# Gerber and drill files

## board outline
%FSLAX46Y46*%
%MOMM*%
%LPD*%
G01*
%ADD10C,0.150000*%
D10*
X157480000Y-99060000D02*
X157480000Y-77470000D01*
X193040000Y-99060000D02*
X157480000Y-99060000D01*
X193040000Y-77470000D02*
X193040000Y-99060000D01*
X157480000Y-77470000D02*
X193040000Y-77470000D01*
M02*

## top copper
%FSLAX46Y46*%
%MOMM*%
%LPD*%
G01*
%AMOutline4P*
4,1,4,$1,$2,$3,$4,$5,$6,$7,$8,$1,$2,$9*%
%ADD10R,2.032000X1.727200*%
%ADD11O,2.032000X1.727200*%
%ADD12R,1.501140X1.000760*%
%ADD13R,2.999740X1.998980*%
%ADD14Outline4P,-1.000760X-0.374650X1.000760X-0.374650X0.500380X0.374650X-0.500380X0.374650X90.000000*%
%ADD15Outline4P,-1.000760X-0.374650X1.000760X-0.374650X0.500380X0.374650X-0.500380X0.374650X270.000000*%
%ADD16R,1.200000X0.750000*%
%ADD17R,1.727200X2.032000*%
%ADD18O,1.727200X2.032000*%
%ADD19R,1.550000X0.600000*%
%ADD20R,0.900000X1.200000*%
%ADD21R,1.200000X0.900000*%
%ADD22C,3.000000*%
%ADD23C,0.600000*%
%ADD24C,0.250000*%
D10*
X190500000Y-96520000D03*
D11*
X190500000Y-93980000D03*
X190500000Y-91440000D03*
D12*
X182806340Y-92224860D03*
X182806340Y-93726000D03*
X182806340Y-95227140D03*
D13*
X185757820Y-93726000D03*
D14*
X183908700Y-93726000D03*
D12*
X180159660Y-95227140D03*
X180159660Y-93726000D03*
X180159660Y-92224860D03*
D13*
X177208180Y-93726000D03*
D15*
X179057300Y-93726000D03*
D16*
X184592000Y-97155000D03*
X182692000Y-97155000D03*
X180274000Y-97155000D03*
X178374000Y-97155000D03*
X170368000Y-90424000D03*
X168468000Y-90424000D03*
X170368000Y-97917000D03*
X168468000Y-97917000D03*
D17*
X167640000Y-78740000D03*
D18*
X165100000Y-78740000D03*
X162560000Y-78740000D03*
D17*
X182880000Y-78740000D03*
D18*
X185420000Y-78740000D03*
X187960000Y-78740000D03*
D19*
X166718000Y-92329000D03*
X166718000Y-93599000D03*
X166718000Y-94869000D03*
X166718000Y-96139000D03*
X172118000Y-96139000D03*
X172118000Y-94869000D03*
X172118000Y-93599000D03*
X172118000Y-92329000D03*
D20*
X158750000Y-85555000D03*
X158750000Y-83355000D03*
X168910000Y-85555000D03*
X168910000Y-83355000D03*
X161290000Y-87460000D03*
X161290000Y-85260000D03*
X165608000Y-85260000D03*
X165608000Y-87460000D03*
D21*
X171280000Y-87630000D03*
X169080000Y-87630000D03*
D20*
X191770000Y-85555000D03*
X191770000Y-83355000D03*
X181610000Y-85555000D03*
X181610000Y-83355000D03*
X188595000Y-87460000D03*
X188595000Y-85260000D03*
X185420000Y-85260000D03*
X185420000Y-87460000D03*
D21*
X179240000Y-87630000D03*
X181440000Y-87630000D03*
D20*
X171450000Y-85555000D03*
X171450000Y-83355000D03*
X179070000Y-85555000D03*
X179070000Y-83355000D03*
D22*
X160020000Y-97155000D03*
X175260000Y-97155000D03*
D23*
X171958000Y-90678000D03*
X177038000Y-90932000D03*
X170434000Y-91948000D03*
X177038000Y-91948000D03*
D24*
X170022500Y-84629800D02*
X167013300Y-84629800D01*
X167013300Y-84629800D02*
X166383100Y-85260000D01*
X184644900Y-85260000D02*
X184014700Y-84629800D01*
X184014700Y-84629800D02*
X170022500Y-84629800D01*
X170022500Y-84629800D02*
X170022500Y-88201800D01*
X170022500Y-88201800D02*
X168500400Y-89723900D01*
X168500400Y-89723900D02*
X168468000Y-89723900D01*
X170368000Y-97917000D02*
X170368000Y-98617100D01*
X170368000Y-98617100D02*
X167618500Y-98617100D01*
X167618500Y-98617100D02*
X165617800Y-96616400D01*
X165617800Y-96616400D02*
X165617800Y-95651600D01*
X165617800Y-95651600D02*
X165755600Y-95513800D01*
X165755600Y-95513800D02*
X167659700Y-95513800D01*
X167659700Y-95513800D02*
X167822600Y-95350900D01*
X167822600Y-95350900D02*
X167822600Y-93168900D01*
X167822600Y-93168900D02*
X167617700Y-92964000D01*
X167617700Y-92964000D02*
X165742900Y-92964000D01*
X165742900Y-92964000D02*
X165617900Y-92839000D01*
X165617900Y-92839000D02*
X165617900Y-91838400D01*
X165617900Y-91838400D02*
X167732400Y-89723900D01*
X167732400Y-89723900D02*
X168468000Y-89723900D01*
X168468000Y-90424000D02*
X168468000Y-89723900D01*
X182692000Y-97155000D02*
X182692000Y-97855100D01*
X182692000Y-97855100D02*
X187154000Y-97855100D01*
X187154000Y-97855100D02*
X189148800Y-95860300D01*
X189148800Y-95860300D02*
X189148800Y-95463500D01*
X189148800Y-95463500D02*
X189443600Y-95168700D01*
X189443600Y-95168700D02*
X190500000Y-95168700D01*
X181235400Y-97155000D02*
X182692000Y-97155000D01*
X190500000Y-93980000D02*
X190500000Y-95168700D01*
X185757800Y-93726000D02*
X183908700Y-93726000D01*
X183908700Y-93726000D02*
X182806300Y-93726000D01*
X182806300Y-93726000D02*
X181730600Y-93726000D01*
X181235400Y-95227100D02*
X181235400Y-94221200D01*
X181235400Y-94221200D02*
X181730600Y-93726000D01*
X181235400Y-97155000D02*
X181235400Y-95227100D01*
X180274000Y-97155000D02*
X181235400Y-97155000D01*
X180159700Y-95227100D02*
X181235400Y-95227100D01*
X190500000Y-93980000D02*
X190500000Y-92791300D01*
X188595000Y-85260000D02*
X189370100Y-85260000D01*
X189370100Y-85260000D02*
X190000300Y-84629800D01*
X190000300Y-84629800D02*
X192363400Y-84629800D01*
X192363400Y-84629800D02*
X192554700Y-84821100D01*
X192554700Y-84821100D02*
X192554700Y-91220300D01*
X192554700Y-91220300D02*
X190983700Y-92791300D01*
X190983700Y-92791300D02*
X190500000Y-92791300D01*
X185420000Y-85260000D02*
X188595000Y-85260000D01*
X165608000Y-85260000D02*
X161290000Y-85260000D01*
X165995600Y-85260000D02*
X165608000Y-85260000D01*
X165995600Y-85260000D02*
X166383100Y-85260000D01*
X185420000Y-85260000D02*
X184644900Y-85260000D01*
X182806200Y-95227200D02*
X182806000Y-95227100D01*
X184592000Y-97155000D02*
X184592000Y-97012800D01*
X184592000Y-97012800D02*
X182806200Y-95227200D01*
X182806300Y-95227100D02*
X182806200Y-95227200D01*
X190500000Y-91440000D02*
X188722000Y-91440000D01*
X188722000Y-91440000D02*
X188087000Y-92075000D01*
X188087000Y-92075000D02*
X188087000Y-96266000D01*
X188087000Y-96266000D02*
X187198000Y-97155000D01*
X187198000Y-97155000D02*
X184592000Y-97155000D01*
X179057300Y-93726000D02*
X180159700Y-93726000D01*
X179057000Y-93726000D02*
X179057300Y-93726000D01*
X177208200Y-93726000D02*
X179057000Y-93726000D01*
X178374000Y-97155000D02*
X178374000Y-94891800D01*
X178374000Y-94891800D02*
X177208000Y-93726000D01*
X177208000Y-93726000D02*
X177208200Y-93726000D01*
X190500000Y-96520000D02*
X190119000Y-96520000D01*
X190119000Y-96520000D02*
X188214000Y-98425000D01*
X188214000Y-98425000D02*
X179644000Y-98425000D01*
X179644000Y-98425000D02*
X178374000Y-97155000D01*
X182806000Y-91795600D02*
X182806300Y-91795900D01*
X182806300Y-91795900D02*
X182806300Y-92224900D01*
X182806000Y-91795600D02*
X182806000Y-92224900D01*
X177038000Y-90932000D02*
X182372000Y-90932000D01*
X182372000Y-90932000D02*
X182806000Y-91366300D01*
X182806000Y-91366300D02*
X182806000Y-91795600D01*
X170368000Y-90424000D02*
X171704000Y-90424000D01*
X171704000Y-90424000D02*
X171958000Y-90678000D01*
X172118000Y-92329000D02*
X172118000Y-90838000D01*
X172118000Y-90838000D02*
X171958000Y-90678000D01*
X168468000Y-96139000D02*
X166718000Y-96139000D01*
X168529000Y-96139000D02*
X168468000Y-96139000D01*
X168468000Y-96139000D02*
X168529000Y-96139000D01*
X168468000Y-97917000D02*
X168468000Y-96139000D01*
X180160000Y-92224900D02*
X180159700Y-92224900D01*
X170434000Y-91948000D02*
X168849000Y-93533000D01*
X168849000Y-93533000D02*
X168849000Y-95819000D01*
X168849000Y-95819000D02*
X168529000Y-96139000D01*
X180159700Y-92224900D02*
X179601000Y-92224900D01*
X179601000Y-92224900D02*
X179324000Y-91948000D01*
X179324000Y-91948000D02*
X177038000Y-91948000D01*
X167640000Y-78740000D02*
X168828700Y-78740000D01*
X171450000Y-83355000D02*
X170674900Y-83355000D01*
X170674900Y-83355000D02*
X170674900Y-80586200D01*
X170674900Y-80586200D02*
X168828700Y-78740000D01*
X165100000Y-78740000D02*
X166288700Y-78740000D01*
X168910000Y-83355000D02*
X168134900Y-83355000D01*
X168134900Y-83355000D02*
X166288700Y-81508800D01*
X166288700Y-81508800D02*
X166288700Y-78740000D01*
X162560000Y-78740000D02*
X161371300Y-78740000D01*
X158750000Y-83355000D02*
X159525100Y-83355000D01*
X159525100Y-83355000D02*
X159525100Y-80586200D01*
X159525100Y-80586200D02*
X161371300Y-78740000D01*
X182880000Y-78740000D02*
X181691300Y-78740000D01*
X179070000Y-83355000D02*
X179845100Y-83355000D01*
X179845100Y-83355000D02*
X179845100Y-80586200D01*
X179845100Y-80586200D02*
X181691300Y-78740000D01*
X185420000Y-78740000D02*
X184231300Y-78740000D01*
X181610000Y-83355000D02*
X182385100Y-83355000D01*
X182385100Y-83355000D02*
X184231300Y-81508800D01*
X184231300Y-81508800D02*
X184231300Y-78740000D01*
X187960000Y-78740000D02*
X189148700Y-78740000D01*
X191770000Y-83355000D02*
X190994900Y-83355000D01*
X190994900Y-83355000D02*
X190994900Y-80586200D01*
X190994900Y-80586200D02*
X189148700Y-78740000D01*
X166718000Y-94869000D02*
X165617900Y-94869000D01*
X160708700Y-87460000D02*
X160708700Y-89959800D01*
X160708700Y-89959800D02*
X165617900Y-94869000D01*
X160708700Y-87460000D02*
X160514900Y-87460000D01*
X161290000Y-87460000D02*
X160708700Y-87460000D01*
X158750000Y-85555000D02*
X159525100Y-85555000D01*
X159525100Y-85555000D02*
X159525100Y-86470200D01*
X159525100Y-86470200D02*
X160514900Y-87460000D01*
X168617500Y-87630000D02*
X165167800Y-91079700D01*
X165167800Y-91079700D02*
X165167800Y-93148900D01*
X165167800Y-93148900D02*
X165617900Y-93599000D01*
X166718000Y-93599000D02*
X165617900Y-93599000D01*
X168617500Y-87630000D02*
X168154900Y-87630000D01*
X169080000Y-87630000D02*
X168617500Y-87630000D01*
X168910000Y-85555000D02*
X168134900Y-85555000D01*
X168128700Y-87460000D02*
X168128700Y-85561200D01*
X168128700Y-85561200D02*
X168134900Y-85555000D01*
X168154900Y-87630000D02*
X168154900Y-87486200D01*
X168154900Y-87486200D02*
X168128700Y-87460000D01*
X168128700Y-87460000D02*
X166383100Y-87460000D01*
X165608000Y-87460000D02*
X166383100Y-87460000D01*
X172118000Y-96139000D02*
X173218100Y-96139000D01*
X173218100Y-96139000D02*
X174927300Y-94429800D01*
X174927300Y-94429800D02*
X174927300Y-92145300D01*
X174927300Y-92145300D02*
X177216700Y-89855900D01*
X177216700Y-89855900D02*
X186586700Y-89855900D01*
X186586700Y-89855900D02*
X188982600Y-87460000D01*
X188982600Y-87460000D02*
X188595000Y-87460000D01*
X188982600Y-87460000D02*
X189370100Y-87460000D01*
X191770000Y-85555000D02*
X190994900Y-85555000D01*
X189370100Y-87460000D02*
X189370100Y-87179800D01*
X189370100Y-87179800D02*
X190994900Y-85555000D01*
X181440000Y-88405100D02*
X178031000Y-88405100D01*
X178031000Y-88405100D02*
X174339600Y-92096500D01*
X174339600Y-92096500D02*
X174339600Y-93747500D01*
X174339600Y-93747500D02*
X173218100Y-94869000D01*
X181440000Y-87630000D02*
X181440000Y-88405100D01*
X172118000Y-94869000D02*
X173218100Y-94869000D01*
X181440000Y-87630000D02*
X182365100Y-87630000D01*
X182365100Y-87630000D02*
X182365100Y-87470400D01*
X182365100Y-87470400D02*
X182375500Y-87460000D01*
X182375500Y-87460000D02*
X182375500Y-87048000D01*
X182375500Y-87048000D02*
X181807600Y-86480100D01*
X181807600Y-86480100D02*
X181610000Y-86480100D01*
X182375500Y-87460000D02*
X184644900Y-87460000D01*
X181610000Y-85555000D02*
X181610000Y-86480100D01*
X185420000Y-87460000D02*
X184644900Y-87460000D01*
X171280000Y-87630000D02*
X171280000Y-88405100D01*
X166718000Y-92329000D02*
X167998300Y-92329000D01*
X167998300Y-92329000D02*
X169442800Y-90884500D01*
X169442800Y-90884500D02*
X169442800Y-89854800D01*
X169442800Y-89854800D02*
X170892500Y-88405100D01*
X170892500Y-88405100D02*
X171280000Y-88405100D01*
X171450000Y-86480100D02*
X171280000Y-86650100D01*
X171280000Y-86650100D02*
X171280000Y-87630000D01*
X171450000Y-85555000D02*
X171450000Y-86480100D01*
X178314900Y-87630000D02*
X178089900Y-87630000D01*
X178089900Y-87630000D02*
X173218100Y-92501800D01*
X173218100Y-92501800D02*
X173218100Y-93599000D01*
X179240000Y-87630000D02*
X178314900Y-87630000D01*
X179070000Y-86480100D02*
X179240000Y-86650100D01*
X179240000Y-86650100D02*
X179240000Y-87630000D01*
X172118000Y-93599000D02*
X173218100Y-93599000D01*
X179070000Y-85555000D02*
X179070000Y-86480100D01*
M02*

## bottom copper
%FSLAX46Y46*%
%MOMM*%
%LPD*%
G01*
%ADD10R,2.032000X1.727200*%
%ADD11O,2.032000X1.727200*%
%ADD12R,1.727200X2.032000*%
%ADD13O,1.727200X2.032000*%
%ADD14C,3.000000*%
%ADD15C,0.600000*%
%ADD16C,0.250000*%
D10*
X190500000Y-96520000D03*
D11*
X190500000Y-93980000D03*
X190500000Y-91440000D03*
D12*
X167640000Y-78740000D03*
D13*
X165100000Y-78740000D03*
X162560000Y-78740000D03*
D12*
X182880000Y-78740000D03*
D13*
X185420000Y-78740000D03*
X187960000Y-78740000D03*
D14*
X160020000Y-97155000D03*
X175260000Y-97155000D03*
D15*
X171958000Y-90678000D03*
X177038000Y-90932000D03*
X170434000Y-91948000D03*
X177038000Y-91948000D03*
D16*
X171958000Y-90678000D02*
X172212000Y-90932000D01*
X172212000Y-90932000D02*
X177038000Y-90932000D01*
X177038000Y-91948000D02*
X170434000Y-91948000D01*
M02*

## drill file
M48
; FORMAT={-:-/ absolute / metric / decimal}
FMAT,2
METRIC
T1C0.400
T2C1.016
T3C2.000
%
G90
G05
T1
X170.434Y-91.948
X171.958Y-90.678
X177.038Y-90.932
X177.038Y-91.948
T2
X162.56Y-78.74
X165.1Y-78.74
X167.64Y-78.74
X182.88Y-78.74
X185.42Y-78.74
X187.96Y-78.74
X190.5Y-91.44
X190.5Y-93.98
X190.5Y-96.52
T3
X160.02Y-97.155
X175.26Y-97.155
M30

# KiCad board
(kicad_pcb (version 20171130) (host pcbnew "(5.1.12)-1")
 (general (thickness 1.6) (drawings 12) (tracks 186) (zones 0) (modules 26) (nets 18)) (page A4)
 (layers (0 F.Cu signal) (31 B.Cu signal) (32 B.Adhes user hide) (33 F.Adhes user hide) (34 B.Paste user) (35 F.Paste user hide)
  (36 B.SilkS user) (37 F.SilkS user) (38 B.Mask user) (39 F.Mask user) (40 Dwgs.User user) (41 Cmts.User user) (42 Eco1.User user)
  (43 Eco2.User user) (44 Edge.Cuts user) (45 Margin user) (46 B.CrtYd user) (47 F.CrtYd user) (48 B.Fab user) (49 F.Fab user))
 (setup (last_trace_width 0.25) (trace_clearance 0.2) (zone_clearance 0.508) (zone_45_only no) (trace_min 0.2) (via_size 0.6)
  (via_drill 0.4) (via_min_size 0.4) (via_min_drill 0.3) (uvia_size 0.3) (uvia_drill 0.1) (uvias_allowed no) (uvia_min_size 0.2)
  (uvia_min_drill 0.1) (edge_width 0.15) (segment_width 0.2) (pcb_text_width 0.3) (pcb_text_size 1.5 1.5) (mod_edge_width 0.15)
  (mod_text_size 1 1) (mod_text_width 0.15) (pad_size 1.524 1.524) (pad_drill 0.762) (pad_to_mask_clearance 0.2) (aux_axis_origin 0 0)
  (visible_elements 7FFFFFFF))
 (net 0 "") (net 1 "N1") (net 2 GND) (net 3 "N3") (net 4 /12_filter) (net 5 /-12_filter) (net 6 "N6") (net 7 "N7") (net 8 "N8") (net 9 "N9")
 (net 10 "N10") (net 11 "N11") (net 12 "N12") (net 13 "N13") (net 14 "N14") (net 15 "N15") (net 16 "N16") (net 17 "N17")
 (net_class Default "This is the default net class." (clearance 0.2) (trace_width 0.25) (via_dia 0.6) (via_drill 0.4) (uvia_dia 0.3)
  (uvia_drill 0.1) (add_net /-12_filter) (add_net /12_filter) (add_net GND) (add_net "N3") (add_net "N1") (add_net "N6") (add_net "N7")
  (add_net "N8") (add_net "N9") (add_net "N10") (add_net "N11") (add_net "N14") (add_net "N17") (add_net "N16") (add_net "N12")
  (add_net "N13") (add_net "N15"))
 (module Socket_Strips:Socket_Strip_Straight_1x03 (layer F.Cu) (at 190.5 96.52 90)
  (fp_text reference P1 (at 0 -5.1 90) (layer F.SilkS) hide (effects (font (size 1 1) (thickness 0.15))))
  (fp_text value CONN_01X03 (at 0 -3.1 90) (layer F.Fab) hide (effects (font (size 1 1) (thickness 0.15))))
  (pad 1 thru_hole rect (at 0 0 90) (size 1.7272 2.032) (drill 1.016) (layers *.Cu *.Mask F.SilkS) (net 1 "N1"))
  (pad 2 thru_hole oval (at 2.54 0 90) (size 1.7272 2.032) (drill 1.016) (layers *.Cu *.Mask F.SilkS) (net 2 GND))
  (pad 3 thru_hole oval (at 5.08 0 90) (size 1.7272 2.032) (drill 1.016) (layers *.Cu *.Mask F.SilkS) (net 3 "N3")))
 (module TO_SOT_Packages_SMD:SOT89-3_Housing (layer F.Cu) (at 184.658 93.726 270)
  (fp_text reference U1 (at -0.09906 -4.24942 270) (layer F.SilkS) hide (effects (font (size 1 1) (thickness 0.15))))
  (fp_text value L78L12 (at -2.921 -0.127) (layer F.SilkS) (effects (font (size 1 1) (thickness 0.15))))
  (pad 1 smd rect (at -1.50114 1.85166 270) (size 1.00076 1.50114) (layers F.Cu F.Paste F.Mask) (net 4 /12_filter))
  (pad 2 smd rect (at 0 1.85166 270) (size 1.00076 1.50114) (layers F.Cu F.Paste F.Mask) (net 2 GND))
  (pad 3 smd rect (at 1.50114 1.85166 270) (size 1.00076 1.50114) (layers F.Cu F.Paste F.Mask) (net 3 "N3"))
  (pad 2 smd rect (at 0 -1.09982 270) (size 1.99898 2.99974) (layers F.Cu F.Paste F.Mask) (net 2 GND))
  (pad 2 smd trapezoid (at 0 0.7493 90) (size 1.50114 0.7493) (rect_delta 0 0.50038) (layers F.Cu F.Paste F.Mask) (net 2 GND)))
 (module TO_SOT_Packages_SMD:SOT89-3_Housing (layer F.Cu) (at 178.308 93.726 90)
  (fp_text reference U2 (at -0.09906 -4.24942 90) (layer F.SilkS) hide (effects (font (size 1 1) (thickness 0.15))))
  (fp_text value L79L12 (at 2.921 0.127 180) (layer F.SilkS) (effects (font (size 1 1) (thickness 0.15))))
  (pad 1 smd rect (at -1.50114 1.85166 90) (size 1.00076 1.50114) (layers F.Cu F.Paste F.Mask) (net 2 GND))
  (pad 2 smd rect (at 0 1.85166 90) (size 1.00076 1.50114) (layers F.Cu F.Paste F.Mask) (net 1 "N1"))
  (pad 3 smd rect (at 1.50114 1.85166 90) (size 1.00076 1.50114) (layers F.Cu F.Paste F.Mask) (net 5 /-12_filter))
  (pad 2 smd rect (at 0 -1.09982 90) (size 1.99898 2.99974) (layers F.Cu F.Paste F.Mask) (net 1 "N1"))
  (pad 2 smd trapezoid (at 0 0.7493 270) (size 1.50114 0.7493) (rect_delta 0 0.50038) (layers F.Cu F.Paste F.Mask) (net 1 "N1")))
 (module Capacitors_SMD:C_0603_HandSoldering (layer F.Cu) (at 183.642 97.155 180)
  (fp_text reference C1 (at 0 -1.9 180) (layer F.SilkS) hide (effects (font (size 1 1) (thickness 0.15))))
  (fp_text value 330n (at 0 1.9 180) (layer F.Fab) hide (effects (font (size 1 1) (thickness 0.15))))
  (pad 1 smd rect (at -0.95 0 180) (size 1.2 0.75) (layers F.Cu F.Paste F.Mask) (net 3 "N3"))
  (pad 2 smd rect (at 0.95 0 180) (size 1.2 0.75) (layers F.Cu F.Paste F.Mask) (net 2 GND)))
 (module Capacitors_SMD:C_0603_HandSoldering (layer F.Cu) (at 179.324 97.155 180)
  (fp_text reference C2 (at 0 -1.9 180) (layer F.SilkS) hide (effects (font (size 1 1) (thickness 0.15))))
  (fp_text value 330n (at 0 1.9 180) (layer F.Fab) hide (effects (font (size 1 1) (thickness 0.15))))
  (pad 1 smd rect (at -0.95 0 180) (size 1.2 0.75) (layers F.Cu F.Paste F.Mask) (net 2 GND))
  (pad 2 smd rect (at 0.95 0 180) (size 1.2 0.75) (layers F.Cu F.Paste F.Mask) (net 1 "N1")))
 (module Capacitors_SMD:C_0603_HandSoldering (layer F.Cu) (at 169.418 90.424 180)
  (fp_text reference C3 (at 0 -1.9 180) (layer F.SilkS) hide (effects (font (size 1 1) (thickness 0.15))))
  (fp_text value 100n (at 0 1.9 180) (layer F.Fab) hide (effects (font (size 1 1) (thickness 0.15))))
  (pad 1 smd rect (at -0.95 0 180) (size 1.2 0.75) (layers F.Cu F.Paste F.Mask) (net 4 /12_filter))
  (pad 2 smd rect (at 0.95 0 180) (size 1.2 0.75) (layers F.Cu F.Paste F.Mask) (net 2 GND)))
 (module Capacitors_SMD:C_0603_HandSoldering (layer F.Cu) (at 169.418 97.917 180)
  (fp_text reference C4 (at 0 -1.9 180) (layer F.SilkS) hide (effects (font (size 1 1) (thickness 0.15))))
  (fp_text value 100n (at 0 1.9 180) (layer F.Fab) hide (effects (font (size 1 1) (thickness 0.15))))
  (pad 1 smd rect (at -0.95 0 180) (size 1.2 0.75) (layers F.Cu F.Paste F.Mask) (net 2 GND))
  (pad 2 smd rect (at 0.95 0 180) (size 1.2 0.75) (layers F.Cu F.Paste F.Mask) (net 5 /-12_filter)))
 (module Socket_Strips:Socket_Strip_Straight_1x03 (layer F.Cu) (at 167.64 78.74 180)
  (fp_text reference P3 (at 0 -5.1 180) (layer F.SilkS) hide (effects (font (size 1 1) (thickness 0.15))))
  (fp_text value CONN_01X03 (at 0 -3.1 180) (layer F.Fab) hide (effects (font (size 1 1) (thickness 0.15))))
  (pad 1 thru_hole rect (at 0 0 180) (size 1.7272 2.032) (drill 1.016) (layers *.Cu *.Mask F.SilkS) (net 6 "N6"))
  (pad 2 thru_hole oval (at 2.54 0 180) (size 1.7272 2.032) (drill 1.016) (layers *.Cu *.Mask F.SilkS) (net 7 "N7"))
  (pad 3 thru_hole oval (at 5.08 0 180) (size 1.7272 2.032) (drill 1.016) (layers *.Cu *.Mask F.SilkS) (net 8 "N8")))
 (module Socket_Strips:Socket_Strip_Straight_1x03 (layer F.Cu) (at 182.88 78.74)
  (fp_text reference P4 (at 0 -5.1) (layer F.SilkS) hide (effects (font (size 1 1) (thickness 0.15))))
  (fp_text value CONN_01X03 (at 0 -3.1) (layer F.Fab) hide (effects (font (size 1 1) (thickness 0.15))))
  (pad 1 thru_hole rect (at 0 0) (size 1.7272 2.032) (drill 1.016) (layers *.Cu *.Mask F.SilkS) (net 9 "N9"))
  (pad 2 thru_hole oval (at 2.54 0) (size 1.7272 2.032) (drill 1.016) (layers *.Cu *.Mask F.SilkS) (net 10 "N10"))
  (pad 3 thru_hole oval (at 5.08 0) (size 1.7272 2.032) (drill 1.016) (layers *.Cu *.Mask F.SilkS) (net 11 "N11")))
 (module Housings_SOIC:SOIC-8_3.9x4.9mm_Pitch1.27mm (layer F.Cu) (at 169.418 94.234)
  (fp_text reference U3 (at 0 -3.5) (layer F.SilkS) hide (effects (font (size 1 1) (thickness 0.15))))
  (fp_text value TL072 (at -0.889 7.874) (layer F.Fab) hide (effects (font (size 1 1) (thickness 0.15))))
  (pad 1 smd rect (at -2.7 -1.905) (size 1.55 0.6) (layers F.Cu F.Paste F.Mask) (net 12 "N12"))
  (pad 2 smd rect (at -2.7 -0.635) (size 1.55 0.6) (layers F.Cu F.Paste F.Mask) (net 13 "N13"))
  (pad 3 smd rect (at -2.7 0.635) (size 1.55 0.6) (layers F.Cu F.Paste F.Mask) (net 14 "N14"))
  (pad 4 smd rect (at -2.7 1.905) (size 1.55 0.6) (layers F.Cu F.Paste F.Mask) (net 5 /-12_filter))
  (pad 5 smd rect (at 2.7 1.905) (size 1.55 0.6) (layers F.Cu F.Paste F.Mask) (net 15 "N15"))
  (pad 6 smd rect (at 2.7 0.635) (size 1.55 0.6) (layers F.Cu F.Paste F.Mask) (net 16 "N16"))
  (pad 7 smd rect (at 2.7 -0.635) (size 1.55 0.6) (layers F.Cu F.Paste F.Mask) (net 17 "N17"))
  (pad 8 smd rect (at 2.7 -1.905) (size 1.55 0.6) (layers F.Cu F.Paste F.Mask) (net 4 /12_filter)))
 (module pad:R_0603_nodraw (layer F.Cu) (at 158.75 84.455 90)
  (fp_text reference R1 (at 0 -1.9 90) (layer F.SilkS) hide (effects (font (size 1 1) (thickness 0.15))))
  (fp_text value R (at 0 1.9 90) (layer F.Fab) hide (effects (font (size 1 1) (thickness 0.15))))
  (pad 1 smd rect (at -1.1 0 90) (size 1.2 0.9) (layers F.Cu F.Paste F.Mask) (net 14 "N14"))
  (pad 2 smd rect (at 1.1 0 90) (size 1.2 0.9) (layers F.Cu F.Paste F.Mask) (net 8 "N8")))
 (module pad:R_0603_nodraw (layer F.Cu) (at 168.91 84.455 90)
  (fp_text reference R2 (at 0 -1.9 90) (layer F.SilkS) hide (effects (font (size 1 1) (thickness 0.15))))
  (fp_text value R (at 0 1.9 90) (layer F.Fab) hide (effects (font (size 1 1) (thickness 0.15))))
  (pad 1 smd rect (at -1.1 0 90) (size 1.2 0.9) (layers F.Cu F.Paste F.Mask) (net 13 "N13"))
  (pad 2 smd rect (at 1.1 0 90) (size 1.2 0.9) (layers F.Cu F.Paste F.Mask) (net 7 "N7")))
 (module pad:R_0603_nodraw (layer F.Cu) (at 161.29 86.36 90)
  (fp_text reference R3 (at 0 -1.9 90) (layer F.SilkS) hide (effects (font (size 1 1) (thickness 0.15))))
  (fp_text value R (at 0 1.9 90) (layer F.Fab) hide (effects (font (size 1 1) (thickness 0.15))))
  (pad 1 smd rect (at -1.1 0 90) (size 1.2 0.9) (layers F.Cu F.Paste F.Mask) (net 14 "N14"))
  (pad 2 smd rect (at 1.1 0 90) (size 1.2 0.9) (layers F.Cu F.Paste F.Mask) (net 2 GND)))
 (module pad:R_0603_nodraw (layer F.Cu) (at 165.608 86.36 270)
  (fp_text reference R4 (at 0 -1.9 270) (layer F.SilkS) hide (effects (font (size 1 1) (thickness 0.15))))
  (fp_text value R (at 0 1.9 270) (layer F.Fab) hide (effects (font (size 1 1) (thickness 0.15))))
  (pad 1 smd rect (at -1.1 0 270) (size 1.2 0.9) (layers F.Cu F.Paste F.Mask) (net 2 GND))
  (pad 2 smd rect (at 1.1 0 270) (size 1.2 0.9) (layers F.Cu F.Paste F.Mask) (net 13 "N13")))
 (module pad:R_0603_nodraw (layer F.Cu) (at 170.18 87.63 180)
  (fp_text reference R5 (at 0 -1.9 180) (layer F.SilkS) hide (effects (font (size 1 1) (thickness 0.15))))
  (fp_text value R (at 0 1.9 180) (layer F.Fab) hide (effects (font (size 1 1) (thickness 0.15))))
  (pad 1 smd rect (at -1.1 0 180) (size 1.2 0.9) (layers F.Cu F.Paste F.Mask) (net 12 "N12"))
  (pad 2 smd rect (at 1.1 0 180) (size 1.2 0.9) (layers F.Cu F.Paste F.Mask) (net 13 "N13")))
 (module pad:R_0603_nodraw (layer F.Cu) (at 191.77 84.455 90)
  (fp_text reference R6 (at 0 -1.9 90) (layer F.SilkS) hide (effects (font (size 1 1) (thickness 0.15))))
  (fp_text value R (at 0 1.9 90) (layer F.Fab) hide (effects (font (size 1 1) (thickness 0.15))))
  (pad 1 smd rect (at -1.1 0 90) (size 1.2 0.9) (layers F.Cu F.Paste F.Mask) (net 15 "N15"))
  (pad 2 smd rect (at 1.1 0 90) (size 1.2 0.9) (layers F.Cu F.Paste F.Mask) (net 11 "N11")))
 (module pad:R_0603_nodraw (layer F.Cu) (at 181.61 84.455 90)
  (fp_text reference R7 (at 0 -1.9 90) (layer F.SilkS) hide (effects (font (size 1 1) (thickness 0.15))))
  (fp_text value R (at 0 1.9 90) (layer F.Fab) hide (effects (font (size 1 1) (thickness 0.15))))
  (pad 1 smd rect (at -1.1 0 90) (size 1.2 0.9) (layers F.Cu F.Paste F.Mask) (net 16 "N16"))
  (pad 2 smd rect (at 1.1 0 90) (size 1.2 0.9) (layers F.Cu F.Paste F.Mask) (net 10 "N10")))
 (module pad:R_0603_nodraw (layer F.Cu) (at 188.595 86.36 90)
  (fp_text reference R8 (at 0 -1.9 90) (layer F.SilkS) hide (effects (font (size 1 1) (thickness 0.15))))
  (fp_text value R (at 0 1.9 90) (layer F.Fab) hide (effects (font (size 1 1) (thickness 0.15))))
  (pad 1 smd rect (at -1.1 0 90) (size 1.2 0.9) (layers F.Cu F.Paste F.Mask) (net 15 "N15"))
  (pad 2 smd rect (at 1.1 0 90) (size 1.2 0.9) (layers F.Cu F.Paste F.Mask) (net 2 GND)))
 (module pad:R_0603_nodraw (layer F.Cu) (at 185.42 86.36 270)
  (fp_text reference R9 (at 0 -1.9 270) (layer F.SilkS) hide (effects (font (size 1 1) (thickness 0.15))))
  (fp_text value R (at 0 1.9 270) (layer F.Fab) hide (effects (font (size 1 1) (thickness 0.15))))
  (pad 1 smd rect (at -1.1 0 270) (size 1.2 0.9) (layers F.Cu F.Paste F.Mask) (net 2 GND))
  (pad 2 smd rect (at 1.1 0 270) (size 1.2 0.9) (layers F.Cu F.Paste F.Mask) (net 16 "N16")))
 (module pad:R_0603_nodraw (layer F.Cu) (at 180.34 87.63)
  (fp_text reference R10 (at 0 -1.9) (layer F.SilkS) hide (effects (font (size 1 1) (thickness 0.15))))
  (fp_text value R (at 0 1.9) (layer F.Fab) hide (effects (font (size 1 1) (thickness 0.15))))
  (pad 1 smd rect (at -1.1 0) (size 1.2 0.9) (layers F.Cu F.Paste F.Mask) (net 17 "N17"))
  (pad 2 smd rect (at 1.1 0) (size 1.2 0.9) (layers F.Cu F.Paste F.Mask) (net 16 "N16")))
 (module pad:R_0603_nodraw (layer F.Cu) (at 171.45 84.455 90)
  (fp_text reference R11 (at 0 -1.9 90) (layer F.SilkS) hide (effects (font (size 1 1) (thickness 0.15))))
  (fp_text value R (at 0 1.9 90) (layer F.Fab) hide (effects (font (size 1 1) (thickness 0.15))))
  (pad 1 smd rect (at -1.1 0 90) (size 1.2 0.9) (layers F.Cu F.Paste F.Mask) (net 12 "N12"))
  (pad 2 smd rect (at 1.1 0 90) (size 1.2 0.9) (layers F.Cu F.Paste F.Mask) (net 6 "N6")))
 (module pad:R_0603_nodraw (layer F.Cu) (at 179.07 84.455 90)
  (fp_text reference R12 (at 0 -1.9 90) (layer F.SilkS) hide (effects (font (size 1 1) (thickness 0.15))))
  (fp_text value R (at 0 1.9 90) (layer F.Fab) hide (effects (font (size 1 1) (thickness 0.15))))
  (pad 1 smd rect (at -1.1 0 90) (size 1.2 0.9) (layers F.Cu F.Paste F.Mask) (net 17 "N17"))
  (pad 2 smd rect (at 1.1 0 90) (size 1.2 0.9) (layers F.Cu F.Paste F.Mask) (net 9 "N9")))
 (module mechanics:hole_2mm (layer F.Cu) (at 160.02 97.155)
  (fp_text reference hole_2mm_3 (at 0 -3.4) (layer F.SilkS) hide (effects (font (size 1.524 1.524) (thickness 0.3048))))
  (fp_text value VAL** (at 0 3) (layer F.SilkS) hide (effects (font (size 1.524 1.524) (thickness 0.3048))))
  (pad 1 thru_hole circle (at 0 0) (size 3 3) (drill 2) (layers *.Cu *.Mask F.SilkS)))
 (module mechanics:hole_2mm (layer F.Cu) (at 175.26 97.155)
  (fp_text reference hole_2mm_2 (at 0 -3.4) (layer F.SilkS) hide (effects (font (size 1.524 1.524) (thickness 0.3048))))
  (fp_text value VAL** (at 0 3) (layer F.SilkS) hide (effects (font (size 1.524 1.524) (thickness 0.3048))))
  (pad 1 thru_hole circle (at 0 0) (size 3 3) (drill 2) (layers *.Cu *.Mask F.SilkS)))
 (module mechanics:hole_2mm (layer F.Cu) (at 196.215 76.2)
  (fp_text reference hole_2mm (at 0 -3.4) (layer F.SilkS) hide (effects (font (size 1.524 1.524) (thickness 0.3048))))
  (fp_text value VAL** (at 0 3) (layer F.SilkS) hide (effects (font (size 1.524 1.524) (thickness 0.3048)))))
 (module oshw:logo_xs (layer F.Cu) (at 162.306 92.964)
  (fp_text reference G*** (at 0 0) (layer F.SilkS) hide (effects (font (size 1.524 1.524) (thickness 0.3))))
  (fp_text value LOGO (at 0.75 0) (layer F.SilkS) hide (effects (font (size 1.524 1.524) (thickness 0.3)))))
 (gr_line (start 157.48 99.06) (end 157.48 77.47) (angle 90) (layer Edge.Cuts) (width 0.15))
 (gr_line (start 193.04 99.06) (end 157.48 99.06) (angle 90) (layer Edge.Cuts) (width 0.15))
 (gr_line (start 193.04 77.47) (end 193.04 99.06) (angle 90) (layer Edge.Cuts) (width 0.15))
 (gr_line (start 157.48 77.47) (end 193.04 77.47) (angle 90) (layer Edge.Cuts) (width 0.15))
 (segment (start 170.0225 84.6298) (end 167.0133 84.6298) (width 0.25) (layer F.Cu) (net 2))
 (segment (start 167.0133 84.6298) (end 166.3831 85.26) (width 0.25) (layer F.Cu) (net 2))
 (segment (start 184.6449 85.26) (end 184.0147 84.6298) (width 0.25) (layer F.Cu) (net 2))
 (segment (start 184.0147 84.6298) (end 170.0225 84.6298) (width 0.25) (layer F.Cu) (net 2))
 (segment (start 170.0225 84.6298) (end 170.0225 88.2018) (width 0.25) (layer F.Cu) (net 2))
 (segment (start 170.0225 88.2018) (end 168.5004 89.7239) (width 0.25) (layer F.Cu) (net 2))
 (segment (start 168.5004 89.7239) (end 168.468 89.7239) (width 0.25) (layer F.Cu) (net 2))
 (segment (start 170.368 97.917) (end 170.368 98.6171) (width 0.25) (layer F.Cu) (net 2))
 (segment (start 170.368 98.6171) (end 167.6185 98.6171) (width 0.25) (layer F.Cu) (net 2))
 (segment (start 167.6185 98.6171) (end 165.6178 96.6164) (width 0.25) (layer F.Cu) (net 2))
 (segment (start 165.6178 96.6164) (end 165.6178 95.6516) (width 0.25) (layer F.Cu) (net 2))
 (segment (start 165.6178 95.6516) (end 165.7556 95.5138) (width 0.25) (layer F.Cu) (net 2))
 (segment (start 165.7556 95.5138) (end 167.6597 95.5138) (width 0.25) (layer F.Cu) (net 2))
 (segment (start 167.6597 95.5138) (end 167.8226 95.3509) (width 0.25) (layer F.Cu) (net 2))
 (segment (start 167.8226 95.3509) (end 167.8226 93.1689) (width 0.25) (layer F.Cu) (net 2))
 (segment (start 167.8226 93.1689) (end 167.6177 92.964) (width 0.25) (layer F.Cu) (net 2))
 (segment (start 167.6177 92.964) (end 165.7429 92.964) (width 0.25) (layer F.Cu) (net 2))
 (segment (start 165.7429 92.964) (end 165.6179 92.839) (width 0.25) (layer F.Cu) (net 2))
 (segment (start 165.6179 92.839) (end 165.6179 91.8384) (width 0.25) (layer F.Cu) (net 2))
 (segment (start 165.6179 91.8384) (end 167.7324 89.7239) (width 0.25) (layer F.Cu) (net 2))
 (segment (start 167.7324 89.7239) (end 168.468 89.7239) (width 0.25) (layer F.Cu) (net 2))
 (segment (start 168.468 90.424) (end 168.468 89.7239) (width 0.25) (layer F.Cu) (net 2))
 (segment (start 182.692 97.155) (end 182.692 97.8551) (width 0.25) (layer F.Cu) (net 2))
 (segment (start 182.692 97.8551) (end 187.154 97.8551) (width 0.25) (layer F.Cu) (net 2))
 (segment (start 187.154 97.8551) (end 189.1488 95.8603) (width 0.25) (layer F.Cu) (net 2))
 (segment (start 189.1488 95.8603) (end 189.1488 95.4635) (width 0.25) (layer F.Cu) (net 2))
 (segment (start 189.1488 95.4635) (end 189.4436 95.1687) (width 0.25) (layer F.Cu) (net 2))
 (segment (start 189.4436 95.1687) (end 190.5 95.1687) (width 0.25) (layer F.Cu) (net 2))
 (segment (start 181.2354 97.155) (end 182.692 97.155) (width 0.25) (layer F.Cu) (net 2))
 (segment (start 190.5 93.98) (end 190.5 95.1687) (width 0.25) (layer F.Cu) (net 2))
 (segment (start 185.7578 93.726) (end 183.9087 93.726) (width 0.25) (layer F.Cu) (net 2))
 (segment (start 183.9087 93.726) (end 182.8063 93.726) (width 0.25) (layer F.Cu) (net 2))
 (segment (start 182.8063 93.726) (end 181.7306 93.726) (width 0.25) (layer F.Cu) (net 2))
 (segment (start 181.2354 95.2271) (end 181.2354 94.2212) (width 0.25) (layer F.Cu) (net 2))
 (segment (start 181.2354 94.2212) (end 181.7306 93.726) (width 0.25) (layer F.Cu) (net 2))
 (segment (start 181.2354 97.155) (end 181.2354 95.2271) (width 0.25) (layer F.Cu) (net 2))
 (segment (start 180.274 97.155) (end 181.2354 97.155) (width 0.25) (layer F.Cu) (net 2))
 (segment (start 180.1597 95.2271) (end 181.2354 95.2271) (width 0.25) (layer F.Cu) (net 2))
 (segment (start 190.5 93.98) (end 190.5 92.7913) (width 0.25) (layer F.Cu) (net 2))
 (segment (start 188.595 85.26) (end 189.3701 85.26) (width 0.25) (layer F.Cu) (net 2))
 (segment (start 189.3701 85.26) (end 190.0003 84.6298) (width 0.25) (layer F.Cu) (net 2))
 (segment (start 190.0003 84.6298) (end 192.3634 84.6298) (width 0.25) (layer F.Cu) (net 2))
 (segment (start 192.3634 84.6298) (end 192.5547 84.8211) (width 0.25) (layer F.Cu) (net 2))
 (segment (start 192.5547 84.8211) (end 192.5547 91.2203) (width 0.25) (layer F.Cu) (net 2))
 (segment (start 192.5547 91.2203) (end 190.9837 92.7913) (width 0.25) (layer F.Cu) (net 2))
 (segment (start 190.9837 92.7913) (end 190.5 92.7913) (width 0.25) (layer F.Cu) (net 2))
 (segment (start 185.42 85.26) (end 188.595 85.26) (width 0.25) (layer F.Cu) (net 2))
 (segment (start 165.608 85.26) (end 161.29 85.26) (width 0.25) (layer F.Cu) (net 2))
 (segment (start 165.9956 85.26) (end 165.608 85.26) (width 0.25) (layer F.Cu) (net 2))
 (segment (start 165.9956 85.26) (end 166.3831 85.26) (width 0.25) (layer F.Cu) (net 2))
 (segment (start 185.42 85.26) (end 184.6449 85.26) (width 0.25) (layer F.Cu) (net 2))
 (segment (start 182.8062 95.2272) (end 182.806 95.2271) (width 0.25) (layer F.Cu) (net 3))
 (segment (start 184.592 97.155) (end 184.592 97.0128) (width 0.25) (layer F.Cu) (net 3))
 (segment (start 184.592 97.0128) (end 182.8062 95.2272) (width 0.25) (layer F.Cu) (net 3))
 (segment (start 182.8063 95.2271) (end 182.8062 95.2272) (width 0.25) (layer F.Cu) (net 3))
 (segment (start 190.5 91.44) (end 188.722 91.44) (width 0.25) (layer F.Cu) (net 3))
 (segment (start 188.722 91.44) (end 188.087 92.075) (width 0.25) (layer F.Cu) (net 3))
 (segment (start 188.087 92.075) (end 188.087 96.266) (width 0.25) (layer F.Cu) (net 3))
 (segment (start 188.087 96.266) (end 187.198 97.155) (width 0.25) (layer F.Cu) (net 3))
 (segment (start 187.198 97.155) (end 184.592 97.155) (width 0.25) (layer F.Cu) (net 3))
 (segment (start 179.0573 93.726) (end 180.1597 93.726) (width 0.25) (layer F.Cu) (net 1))
 (segment (start 179.057 93.726) (end 179.0573 93.726) (width 0.25) (layer F.Cu) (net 1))
 (segment (start 177.2082 93.726) (end 179.057 93.726) (width 0.25) (layer F.Cu) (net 1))
 (segment (start 178.374 97.155) (end 178.374 94.8918) (width 0.25) (layer F.Cu) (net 1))
 (segment (start 178.374 94.8918) (end 177.208 93.726) (width 0.25) (layer F.Cu) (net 1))
 (segment (start 177.208 93.726) (end 177.2082 93.726) (width 0.25) (layer F.Cu) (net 1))
 (segment (start 190.5 96.52) (end 190.119 96.52) (width 0.25) (layer F.Cu) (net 1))
 (segment (start 190.119 96.52) (end 188.214 98.425) (width 0.25) (layer F.Cu) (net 1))
 (segment (start 188.214 98.425) (end 179.644 98.425) (width 0.25) (layer F.Cu) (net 1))
 (segment (start 179.644 98.425) (end 178.374 97.155) (width 0.25) (layer F.Cu) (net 1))
 (segment (start 182.806 91.7956) (end 182.8063 91.7959) (width 0.25) (layer F.Cu) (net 4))
 (segment (start 182.8063 91.7959) (end 182.8063 92.2249) (width 0.25) (layer F.Cu) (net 4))
 (segment (start 182.806 91.7956) (end 182.806 92.2249) (width 0.25) (layer F.Cu) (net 4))
 (segment (start 177.038 90.932) (end 182.372 90.932) (width 0.25) (layer F.Cu) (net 4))
 (segment (start 182.372 90.932) (end 182.806 91.3663) (width 0.25) (layer F.Cu) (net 4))
 (segment (start 182.806 91.3663) (end 182.806 91.7956) (width 0.25) (layer F.Cu) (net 4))
 (segment (start 170.368 90.424) (end 171.704 90.424) (width 0.25) (layer F.Cu) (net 4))
 (segment (start 171.704 90.424) (end 171.958 90.678) (width 0.25) (layer F.Cu) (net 4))
 (segment (start 171.958 90.678) (end 172.212 90.932) (width 0.25) (layer B.Cu) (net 4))
 (segment (start 172.212 90.932) (end 177.038 90.932) (width 0.25) (layer B.Cu) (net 4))
 (segment (start 172.118 92.329) (end 172.118 90.838) (width 0.25) (layer F.Cu) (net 4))
 (segment (start 172.118 90.838) (end 171.958 90.678) (width 0.25) (layer F.Cu) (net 4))
 (via (at 171.958 90.678) (size 0.6) (layers F.Cu B.Cu) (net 4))
 (via (at 177.038 90.932) (size 0.6) (layers F.Cu B.Cu) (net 4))
 (segment (start 168.468 96.139) (end 166.718 96.139) (width 0.25) (layer F.Cu) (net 5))
 (segment (start 168.529 96.139) (end 168.468 96.139) (width 0.25) (layer F.Cu) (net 5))
 (segment (start 168.468 96.139) (end 168.529 96.139) (width 0.25) (layer F.Cu) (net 5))
 (segment (start 168.468 97.917) (end 168.468 96.139) (width 0.25) (layer F.Cu) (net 5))
 (segment (start 180.16 92.2249) (end 180.1597 92.2249) (width 0.25) (layer F.Cu) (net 5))
 (segment (start 170.434 91.948) (end 168.849 93.533) (width 0.25) (layer F.Cu) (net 5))
 (segment (start 168.849 93.533) (end 168.849 95.819) (width 0.25) (layer F.Cu) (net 5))
 (segment (start 168.849 95.819) (end 168.529 96.139) (width 0.25) (layer F.Cu) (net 5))
 (segment (start 177.038 91.948) (end 170.434 91.948) (width 0.25) (layer B.Cu) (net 5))
 (segment (start 180.1597 92.2249) (end 179.601 92.2249) (width 0.25) (layer F.Cu) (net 5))
 (segment (start 179.601 92.2249) (end 179.324 91.948) (width 0.25) (layer F.Cu) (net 5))
 (segment (start 179.324 91.948) (end 177.038 91.948) (width 0.25) (layer F.Cu) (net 5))
 (via (at 170.434 91.948) (size 0.6) (layers F.Cu B.Cu) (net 5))
 (via (at 177.038 91.948) (size 0.6) (layers F.Cu B.Cu) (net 5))
 (segment (start 167.64 78.74) (end 168.8287 78.74) (width 0.25) (layer F.Cu) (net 6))
 (segment (start 171.45 83.355) (end 170.6749 83.355) (width 0.25) (layer F.Cu) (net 6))
 (segment (start 170.6749 83.355) (end 170.6749 80.5862) (width 0.25) (layer F.Cu) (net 6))
 (segment (start 170.6749 80.5862) (end 168.8287 78.74) (width 0.25) (layer F.Cu) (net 6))
 (segment (start 165.1 78.74) (end 166.2887 78.74) (width 0.25) (layer F.Cu) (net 7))
 (segment (start 168.91 83.355) (end 168.1349 83.355) (width 0.25) (layer F.Cu) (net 7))
 (segment (start 168.1349 83.355) (end 166.2887 81.5088) (width 0.25) (layer F.Cu) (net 7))
 (segment (start 166.2887 81.5088) (end 166.2887 78.74) (width 0.25) (layer F.Cu) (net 7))
 (segment (start 162.56 78.74) (end 161.3713 78.74) (width 0.25) (layer F.Cu) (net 8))
 (segment (start 158.75 83.355) (end 159.5251 83.355) (width 0.25) (layer F.Cu) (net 8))
 (segment (start 159.5251 83.355) (end 159.5251 80.5862) (width 0.25) (layer F.Cu) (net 8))
 (segment (start 159.5251 80.5862) (end 161.3713 78.74) (width 0.25) (layer F.Cu) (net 8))
 (segment (start 182.88 78.74) (end 181.6913 78.74) (width 0.25) (layer F.Cu) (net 9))
 (segment (start 179.07 83.355) (end 179.8451 83.355) (width 0.25) (layer F.Cu) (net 9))
 (segment (start 179.8451 83.355) (end 179.8451 80.5862) (width 0.25) (layer F.Cu) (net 9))
 (segment (start 179.8451 80.5862) (end 181.6913 78.74) (width 0.25) (layer F.Cu) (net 9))
 (segment (start 185.42 78.74) (end 184.2313 78.74) (width 0.25) (layer F.Cu) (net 10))
 (segment (start 181.61 83.355) (end 182.3851 83.355) (width 0.25) (layer F.Cu) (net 10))
 (segment (start 182.3851 83.355) (end 184.2313 81.5088) (width 0.25) (layer F.Cu) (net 10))
 (segment (start 184.2313 81.5088) (end 184.2313 78.74) (width 0.25) (layer F.Cu) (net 10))
 (segment (start 187.96 78.74) (end 189.1487 78.74) (width 0.25) (layer F.Cu) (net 11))
 (segment (start 191.77 83.355) (end 190.9949 83.355) (width 0.25) (layer F.Cu) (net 11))
 (segment (start 190.9949 83.355) (end 190.9949 80.5862) (width 0.25) (layer F.Cu) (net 11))
 (segment (start 190.9949 80.5862) (end 189.1487 78.74) (width 0.25) (layer F.Cu) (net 11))
 (segment (start 166.718 94.869) (end 165.6179 94.869) (width 0.25) (layer F.Cu) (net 14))
 (segment (start 160.7087 87.46) (end 160.7087 89.9598) (width 0.25) (layer F.Cu) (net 14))
 (segment (start 160.7087 89.9598) (end 165.6179 94.869) (width 0.25) (layer F.Cu) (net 14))
 (segment (start 160.7087 87.46) (end 160.5149 87.46) (width 0.25) (layer F.Cu) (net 14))
 (segment (start 161.29 87.46) (end 160.7087 87.46) (width 0.25) (layer F.Cu) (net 14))
 (segment (start 158.75 85.555) (end 159.5251 85.555) (width 0.25) (layer F.Cu) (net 14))
 (segment (start 159.5251 85.555) (end 159.5251 86.4702) (width 0.25) (layer F.Cu) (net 14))
 (segment (start 159.5251 86.4702) (end 160.5149 87.46) (width 0.25) (layer F.Cu) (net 14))
 (segment (start 168.6175 87.63) (end 165.1678 91.0797) (width 0.25) (layer F.Cu) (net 13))
 (segment (start 165.1678 91.0797) (end 165.1678 93.1489) (width 0.25) (layer F.Cu) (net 13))
 (segment (start 165.1678 93.1489) (end 165.6179 93.599) (width 0.25) (layer F.Cu) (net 13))
 (segment (start 166.718 93.599) (end 165.6179 93.599) (width 0.25) (layer F.Cu) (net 13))
 (segment (start 168.6175 87.63) (end 168.1549 87.63) (width 0.25) (layer F.Cu) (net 13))
 (segment (start 169.08 87.63) (end 168.6175 87.63) (width 0.25) (layer F.Cu) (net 13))
 (segment (start 168.91 85.555) (end 168.1349 85.555) (width 0.25) (layer F.Cu) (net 13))
 (segment (start 168.1287 87.46) (end 168.1287 85.5612) (width 0.25) (layer F.Cu) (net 13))
 (segment (start 168.1287 85.5612) (end 168.1349 85.555) (width 0.25) (layer F.Cu) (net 13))
 (segment (start 168.1549 87.63) (end 168.1549 87.4862) (width 0.25) (layer F.Cu) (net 13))
 (segment (start 168.1549 87.4862) (end 168.1287 87.46) (width 0.25) (layer F.Cu) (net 13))
 (segment (start 168.1287 87.46) (end 166.3831 87.46) (width 0.25) (layer F.Cu) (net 13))
 (segment (start 165.608 87.46) (end 166.3831 87.46) (width 0.25) (layer F.Cu) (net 13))
 (segment (start 172.118 96.139) (end 173.2181 96.139) (width 0.25) (layer F.Cu) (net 15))
 (segment (start 173.2181 96.139) (end 174.9273 94.4298) (width 0.25) (layer F.Cu) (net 15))
 (segment (start 174.9273 94.4298) (end 174.9273 92.1453) (width 0.25) (layer F.Cu) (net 15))
 (segment (start 174.9273 92.1453) (end 177.2167 89.8559) (width 0.25) (layer F.Cu) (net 15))
 (segment (start 177.2167 89.8559) (end 186.5867 89.8559) (width 0.25) (layer F.Cu) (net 15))
 (segment (start 186.5867 89.8559) (end 188.9826 87.46) (width 0.25) (layer F.Cu) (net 15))
 (segment (start 188.9826 87.46) (end 188.595 87.46) (width 0.25) (layer F.Cu) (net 15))
 (segment (start 188.9826 87.46) (end 189.3701 87.46) (width 0.25) (layer F.Cu) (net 15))
 (segment (start 191.77 85.555) (end 190.9949 85.555) (width 0.25) (layer F.Cu) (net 15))
 (segment (start 189.3701 87.46) (end 189.3701 87.1798) (width 0.25) (layer F.Cu) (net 15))
 (segment (start 189.3701 87.1798) (end 190.9949 85.555) (width 0.25) (layer F.Cu) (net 15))
 (segment (start 181.44 88.4051) (end 178.031 88.4051) (width 0.25) (layer F.Cu) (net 16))
 (segment (start 178.031 88.4051) (end 174.3396 92.0965) (width 0.25) (layer F.Cu) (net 16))
 (segment (start 174.3396 92.0965) (end 174.3396 93.7475) (width 0.25) (layer F.Cu) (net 16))
 (segment (start 174.3396 93.7475) (end 173.2181 94.869) (width 0.25) (layer F.Cu) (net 16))
 (segment (start 181.44 87.63) (end 181.44 88.4051) (width 0.25) (layer F.Cu) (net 16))
 (segment (start 172.118 94.869) (end 173.2181 94.869) (width 0.25) (layer F.Cu) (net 16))
 (segment (start 181.44 87.63) (end 182.3651 87.63) (width 0.25) (layer F.Cu) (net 16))
 (segment (start 182.3651 87.63) (end 182.3651 87.4704) (width 0.25) (layer F.Cu) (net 16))
 (segment (start 182.3651 87.4704) (end 182.3755 87.46) (width 0.25) (layer F.Cu) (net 16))
 (segment (start 182.3755 87.46) (end 182.3755 87.048) (width 0.25) (layer F.Cu) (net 16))
 (segment (start 182.3755 87.048) (end 181.8076 86.4801) (width 0.25) (layer F.Cu) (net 16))
 (segment (start 181.8076 86.4801) (end 181.61 86.4801) (width 0.25) (layer F.Cu) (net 16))
 (segment (start 182.3755 87.46) (end 184.6449 87.46) (width 0.25) (layer F.Cu) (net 16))
 (segment (start 181.61 85.555) (end 181.61 86.4801) (width 0.25) (layer F.Cu) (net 16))
 (segment (start 185.42 87.46) (end 184.6449 87.46) (width 0.25) (layer F.Cu) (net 16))
 (segment (start 171.28 87.63) (end 171.28 88.4051) (width 0.25) (layer F.Cu) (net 12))
 (segment (start 166.718 92.329) (end 167.9983 92.329) (width 0.25) (layer F.Cu) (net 12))
 (segment (start 167.9983 92.329) (end 169.4428 90.8845) (width 0.25) (layer F.Cu) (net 12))
 (segment (start 169.4428 90.8845) (end 169.4428 89.8548) (width 0.25) (layer F.Cu) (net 12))
 (segment (start 169.4428 89.8548) (end 170.8925 88.4051) (width 0.25) (layer F.Cu) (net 12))
 (segment (start 170.8925 88.4051) (end 171.28 88.4051) (width 0.25) (layer F.Cu) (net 12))
 (segment (start 171.45 86.4801) (end 171.28 86.6501) (width 0.25) (layer F.Cu) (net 12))
 (segment (start 171.28 86.6501) (end 171.28 87.63) (width 0.25) (layer F.Cu) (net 12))
 (segment (start 171.45 85.555) (end 171.45 86.4801) (width 0.25) (layer F.Cu) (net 12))
 (segment (start 178.3149 87.63) (end 178.0899 87.63) (width 0.25) (layer F.Cu) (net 17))
 (segment (start 178.0899 87.63) (end 173.2181 92.5018) (width 0.25) (layer F.Cu) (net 17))
 (segment (start 173.2181 92.5018) (end 173.2181 93.599) (width 0.25) (layer F.Cu) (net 17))
 (segment (start 179.24 87.63) (end 178.3149 87.63) (width 0.25) (layer F.Cu) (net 17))
 (segment (start 179.07 86.4801) (end 179.24 86.6501) (width 0.25) (layer F.Cu) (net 17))
 (segment (start 179.24 86.6501) (end 179.24 87.63) (width 0.25) (layer F.Cu) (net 17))
 (segment (start 172.118 93.599) (end 173.2181 93.599) (width 0.25) (layer F.Cu) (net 17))
 (segment (start 179.07 85.555) (end 179.07 86.4801) (width 0.25) (layer F.Cu) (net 17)))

